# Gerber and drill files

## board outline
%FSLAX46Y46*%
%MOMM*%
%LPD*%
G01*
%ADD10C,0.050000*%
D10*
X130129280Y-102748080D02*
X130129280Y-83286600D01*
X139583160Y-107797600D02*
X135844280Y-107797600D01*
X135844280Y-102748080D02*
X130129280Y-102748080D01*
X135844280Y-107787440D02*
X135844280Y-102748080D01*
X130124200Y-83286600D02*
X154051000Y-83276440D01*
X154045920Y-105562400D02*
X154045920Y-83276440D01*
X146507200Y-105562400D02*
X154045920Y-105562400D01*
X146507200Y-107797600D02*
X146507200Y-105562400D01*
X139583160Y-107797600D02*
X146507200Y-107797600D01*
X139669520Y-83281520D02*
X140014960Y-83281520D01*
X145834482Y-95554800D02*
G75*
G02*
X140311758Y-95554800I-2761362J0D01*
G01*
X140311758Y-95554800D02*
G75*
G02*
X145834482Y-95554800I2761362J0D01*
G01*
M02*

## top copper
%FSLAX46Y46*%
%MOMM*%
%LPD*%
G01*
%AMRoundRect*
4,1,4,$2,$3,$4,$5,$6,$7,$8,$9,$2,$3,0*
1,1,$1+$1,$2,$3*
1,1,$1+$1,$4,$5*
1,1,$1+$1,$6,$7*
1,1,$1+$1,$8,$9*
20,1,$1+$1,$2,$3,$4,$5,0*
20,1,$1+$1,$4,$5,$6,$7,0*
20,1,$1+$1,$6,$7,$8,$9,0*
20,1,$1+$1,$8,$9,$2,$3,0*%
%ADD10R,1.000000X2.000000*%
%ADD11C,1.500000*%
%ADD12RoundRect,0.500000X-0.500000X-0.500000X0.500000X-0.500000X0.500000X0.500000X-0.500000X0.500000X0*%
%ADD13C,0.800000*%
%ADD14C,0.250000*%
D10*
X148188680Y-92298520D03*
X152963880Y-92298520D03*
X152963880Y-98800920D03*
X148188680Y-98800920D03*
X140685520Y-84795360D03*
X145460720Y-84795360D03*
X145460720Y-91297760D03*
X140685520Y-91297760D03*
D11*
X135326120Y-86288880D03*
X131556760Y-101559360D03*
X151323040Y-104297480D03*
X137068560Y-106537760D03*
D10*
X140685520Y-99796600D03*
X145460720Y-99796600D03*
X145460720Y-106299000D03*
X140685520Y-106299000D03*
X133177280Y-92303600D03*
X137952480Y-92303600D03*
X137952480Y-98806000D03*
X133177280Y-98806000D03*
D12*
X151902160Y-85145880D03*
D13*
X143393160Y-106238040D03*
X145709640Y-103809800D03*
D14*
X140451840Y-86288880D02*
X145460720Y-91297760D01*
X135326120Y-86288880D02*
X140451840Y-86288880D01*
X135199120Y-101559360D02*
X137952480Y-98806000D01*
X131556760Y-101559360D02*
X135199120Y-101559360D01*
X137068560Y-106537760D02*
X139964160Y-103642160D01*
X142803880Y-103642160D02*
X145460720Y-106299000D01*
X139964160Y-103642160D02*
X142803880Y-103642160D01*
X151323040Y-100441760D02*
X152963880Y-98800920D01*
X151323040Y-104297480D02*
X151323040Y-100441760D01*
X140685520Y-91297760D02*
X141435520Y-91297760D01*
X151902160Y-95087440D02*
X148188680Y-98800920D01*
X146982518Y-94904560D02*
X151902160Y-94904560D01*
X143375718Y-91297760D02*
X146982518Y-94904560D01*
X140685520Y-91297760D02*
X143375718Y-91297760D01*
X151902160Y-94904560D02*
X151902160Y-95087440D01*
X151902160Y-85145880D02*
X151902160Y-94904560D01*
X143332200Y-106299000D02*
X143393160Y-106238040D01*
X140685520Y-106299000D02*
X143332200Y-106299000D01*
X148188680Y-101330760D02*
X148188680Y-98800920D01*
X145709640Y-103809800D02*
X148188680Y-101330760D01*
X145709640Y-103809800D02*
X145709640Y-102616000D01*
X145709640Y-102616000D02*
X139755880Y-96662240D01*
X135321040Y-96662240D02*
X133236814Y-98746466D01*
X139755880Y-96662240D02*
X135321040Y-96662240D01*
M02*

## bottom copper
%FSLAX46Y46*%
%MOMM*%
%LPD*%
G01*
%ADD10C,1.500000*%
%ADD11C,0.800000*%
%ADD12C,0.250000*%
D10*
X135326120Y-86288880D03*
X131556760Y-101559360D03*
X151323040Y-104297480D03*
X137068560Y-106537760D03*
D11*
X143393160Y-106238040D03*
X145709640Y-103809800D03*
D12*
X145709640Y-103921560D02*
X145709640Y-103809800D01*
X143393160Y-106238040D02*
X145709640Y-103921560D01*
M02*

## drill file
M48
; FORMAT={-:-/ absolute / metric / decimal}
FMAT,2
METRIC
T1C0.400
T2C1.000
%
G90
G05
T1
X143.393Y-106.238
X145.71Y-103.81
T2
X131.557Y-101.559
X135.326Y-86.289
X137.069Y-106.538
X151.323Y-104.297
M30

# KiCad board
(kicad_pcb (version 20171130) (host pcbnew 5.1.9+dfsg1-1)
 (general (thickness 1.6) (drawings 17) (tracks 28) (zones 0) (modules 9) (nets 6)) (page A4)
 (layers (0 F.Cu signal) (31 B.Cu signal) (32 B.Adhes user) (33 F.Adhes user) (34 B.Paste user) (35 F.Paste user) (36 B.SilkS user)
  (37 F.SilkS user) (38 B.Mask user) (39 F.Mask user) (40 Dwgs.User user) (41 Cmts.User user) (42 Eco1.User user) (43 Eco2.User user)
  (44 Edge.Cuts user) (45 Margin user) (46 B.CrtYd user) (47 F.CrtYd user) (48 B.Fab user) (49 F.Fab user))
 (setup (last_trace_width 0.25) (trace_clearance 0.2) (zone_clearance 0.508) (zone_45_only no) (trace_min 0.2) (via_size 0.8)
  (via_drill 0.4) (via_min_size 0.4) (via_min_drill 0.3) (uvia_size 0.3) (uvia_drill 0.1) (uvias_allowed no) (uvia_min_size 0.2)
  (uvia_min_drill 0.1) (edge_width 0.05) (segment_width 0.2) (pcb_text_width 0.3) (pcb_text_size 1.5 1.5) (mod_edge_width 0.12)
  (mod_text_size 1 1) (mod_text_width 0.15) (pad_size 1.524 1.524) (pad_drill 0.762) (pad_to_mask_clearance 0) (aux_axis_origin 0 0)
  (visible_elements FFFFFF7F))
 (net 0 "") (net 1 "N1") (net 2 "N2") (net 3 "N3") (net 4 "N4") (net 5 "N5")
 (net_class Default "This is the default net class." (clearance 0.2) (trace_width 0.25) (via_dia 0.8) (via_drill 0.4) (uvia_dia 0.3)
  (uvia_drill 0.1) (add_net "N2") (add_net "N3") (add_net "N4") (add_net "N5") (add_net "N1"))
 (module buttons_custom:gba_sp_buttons (layer F.Cu) (at 150.57628 95.54972)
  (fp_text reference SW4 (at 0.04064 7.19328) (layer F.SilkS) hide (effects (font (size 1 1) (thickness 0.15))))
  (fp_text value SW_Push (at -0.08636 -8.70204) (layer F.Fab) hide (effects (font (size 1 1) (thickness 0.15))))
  (pad 3 smd rect (at -2.3876 -3.2512) (size 1 2) (layers F.Cu F.Paste F.Mask))
  (pad 4 smd rect (at 2.3876 -3.2512) (size 1 2) (layers F.Cu F.Paste F.Mask))
  (pad 2 smd rect (at 2.3876 3.2512) (size 1 2) (layers F.Cu F.Paste F.Mask) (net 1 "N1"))
  (pad 1 smd rect (at -2.3876 3.2512) (size 1 2) (layers F.Cu F.Paste F.Mask) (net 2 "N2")))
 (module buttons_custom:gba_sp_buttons (layer F.Cu) (at 143.07312 88.04656)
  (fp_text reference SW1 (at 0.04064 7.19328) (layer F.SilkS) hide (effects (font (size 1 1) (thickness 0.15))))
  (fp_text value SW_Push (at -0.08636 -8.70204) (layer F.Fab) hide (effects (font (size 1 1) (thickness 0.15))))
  (pad 3 smd rect (at -2.3876 -3.2512) (size 1 2) (layers F.Cu F.Paste F.Mask))
  (pad 4 smd rect (at 2.3876 -3.2512) (size 1 2) (layers F.Cu F.Paste F.Mask))
  (pad 2 smd rect (at 2.3876 3.2512) (size 1 2) (layers F.Cu F.Paste F.Mask) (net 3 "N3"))
  (pad 1 smd rect (at -2.3876 3.2512) (size 1 2) (layers F.Cu F.Paste F.Mask) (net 2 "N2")))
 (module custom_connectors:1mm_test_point (layer F.Cu) (at 135.32612 86.29904)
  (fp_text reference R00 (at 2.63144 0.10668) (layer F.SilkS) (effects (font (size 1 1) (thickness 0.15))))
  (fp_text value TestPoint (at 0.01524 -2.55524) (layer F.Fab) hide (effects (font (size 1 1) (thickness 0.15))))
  (pad 1 thru_hole circle (at 0 -0.01016) (size 1.5 1.5) (drill 1) (layers *.Cu *.Mask) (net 3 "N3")))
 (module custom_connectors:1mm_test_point (layer F.Cu) (at 131.55676 101.56952)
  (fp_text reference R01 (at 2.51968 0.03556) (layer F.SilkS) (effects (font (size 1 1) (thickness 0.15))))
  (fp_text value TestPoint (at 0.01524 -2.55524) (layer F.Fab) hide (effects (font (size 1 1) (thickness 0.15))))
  (pad 1 thru_hole circle (at 0 -0.01016) (size 1.5 1.5) (drill 1) (layers *.Cu *.Mask) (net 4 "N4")))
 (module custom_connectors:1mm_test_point (layer F.Cu) (at 151.32304 104.30764)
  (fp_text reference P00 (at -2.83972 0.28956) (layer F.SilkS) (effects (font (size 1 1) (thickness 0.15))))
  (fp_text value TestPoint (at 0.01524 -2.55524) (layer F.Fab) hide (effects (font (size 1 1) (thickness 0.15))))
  (pad 1 thru_hole circle (at 0 -0.01016) (size 1.5 1.5) (drill 1) (layers *.Cu *.Mask) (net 1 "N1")))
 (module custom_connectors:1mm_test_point (layer F.Cu) (at 137.06856 106.54792)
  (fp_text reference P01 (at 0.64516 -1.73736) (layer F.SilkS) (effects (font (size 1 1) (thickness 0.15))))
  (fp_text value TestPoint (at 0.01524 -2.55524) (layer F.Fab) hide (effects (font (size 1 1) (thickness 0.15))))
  (pad 1 thru_hole circle (at 0 -0.01016) (size 1.5 1.5) (drill 1) (layers *.Cu *.Mask) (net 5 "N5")))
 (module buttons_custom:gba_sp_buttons (layer F.Cu) (at 143.07312 103.0478)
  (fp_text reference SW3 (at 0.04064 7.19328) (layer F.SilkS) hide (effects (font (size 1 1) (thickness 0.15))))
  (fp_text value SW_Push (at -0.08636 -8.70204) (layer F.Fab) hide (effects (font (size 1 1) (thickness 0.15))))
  (pad 3 smd rect (at -2.3876 -3.2512) (size 1 2) (layers F.Cu F.Paste F.Mask))
  (pad 4 smd rect (at 2.3876 -3.2512) (size 1 2) (layers F.Cu F.Paste F.Mask))
  (pad 2 smd rect (at 2.3876 3.2512) (size 1 2) (layers F.Cu F.Paste F.Mask) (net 5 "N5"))
  (pad 1 smd rect (at -2.3876 3.2512) (size 1 2) (layers F.Cu F.Paste F.Mask) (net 2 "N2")))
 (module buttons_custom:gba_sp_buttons (layer F.Cu) (at 135.56488 95.5548)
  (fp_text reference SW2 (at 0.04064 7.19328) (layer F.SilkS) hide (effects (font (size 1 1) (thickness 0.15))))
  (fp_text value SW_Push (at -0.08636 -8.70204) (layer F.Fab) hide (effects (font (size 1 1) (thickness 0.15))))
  (pad 3 smd rect (at -2.3876 -3.2512) (size 1 2) (layers F.Cu F.Paste F.Mask))
  (pad 4 smd rect (at 2.3876 -3.2512) (size 1 2) (layers F.Cu F.Paste F.Mask))
  (pad 2 smd rect (at 2.3876 3.2512) (size 1 2) (layers F.Cu F.Paste F.Mask) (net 4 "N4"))
  (pad 1 smd rect (at -2.3876 3.2512) (size 1 2) (layers F.Cu F.Paste F.Mask) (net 2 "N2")))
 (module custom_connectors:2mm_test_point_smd (layer F.Cu) (at 151.90216 85.15604)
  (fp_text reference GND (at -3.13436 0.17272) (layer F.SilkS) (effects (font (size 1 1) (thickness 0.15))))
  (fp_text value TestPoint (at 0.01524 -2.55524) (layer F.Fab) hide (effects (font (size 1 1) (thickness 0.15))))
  (pad 1 smd roundrect (at 0 -0.01016) (size 2 2) (layers F.Cu F.Paste F.Mask) (roundrect_rratio 0.25) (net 2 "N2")))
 (gr_line (start 130.12928 102.74808) (end 130.12928 83.2866) (layer Edge.Cuts) (width 0.05))
 (gr_line (start 139.58316 107.7976) (end 135.84428 107.7976) (layer Edge.Cuts) (width 0.05))
 (gr_line (start 135.84428 102.74808) (end 130.12928 102.74808) (layer Edge.Cuts) (width 0.05))
 (gr_line (start 135.84428 107.78744) (end 135.84428 102.74808) (layer Edge.Cuts) (width 0.05))
 (gr_line (start 130.1242 83.2866) (end 154.051 83.27644) (layer Edge.Cuts) (width 0.05))
 (gr_line (start 154.04592 105.5624) (end 154.04592 83.27644) (layer Edge.Cuts) (width 0.05))
 (gr_line (start 146.5072 105.5624) (end 154.04592 105.5624) (layer Edge.Cuts) (width 0.05))
 (gr_line (start 146.5072 107.7976) (end 146.5072 105.5624) (layer Edge.Cuts) (width 0.05))
 (gr_line (start 139.58316 107.7976) (end 146.5072 107.7976) (layer Edge.Cuts) (width 0.05))
 (gr_line (start 139.66952 83.28152) (end 140.01496 83.28152) (layer Edge.Cuts) (width 0.05))
 (gr_circle (center 143.07312 95.5548) (end 145.83156 95.4278) (layer Edge.Cuts) (width 0.05))
 (segment (start 140.45184 86.28888) (end 145.46072 91.29776) (width 0.25) (layer F.Cu) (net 3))
 (segment (start 135.32612 86.28888) (end 140.45184 86.28888) (width 0.25) (layer F.Cu) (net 3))
 (segment (start 135.19912 101.55936) (end 137.95248 98.806) (width 0.25) (layer F.Cu) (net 4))
 (segment (start 131.55676 101.55936) (end 135.19912 101.55936) (width 0.25) (layer F.Cu) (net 4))
 (segment (start 137.06856 106.53776) (end 139.96416 103.64216) (width 0.25) (layer F.Cu) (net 5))
 (segment (start 142.80388 103.64216) (end 145.46072 106.299) (width 0.25) (layer F.Cu) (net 5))
 (segment (start 139.96416 103.64216) (end 142.80388 103.64216) (width 0.25) (layer F.Cu) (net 5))
 (segment (start 151.32304 100.44176) (end 152.96388 98.80092) (width 0.25) (layer F.Cu) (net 1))
 (segment (start 151.32304 104.29748) (end 151.32304 100.44176) (width 0.25) (layer F.Cu) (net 1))
 (segment (start 140.68552 91.29776) (end 141.43552 91.29776) (width 0.25) (layer F.Cu) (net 2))
 (segment (start 151.90216 95.08744) (end 148.18868 98.80092) (width 0.25) (layer F.Cu) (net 2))
 (segment (start 146.982518 94.90456) (end 151.90216 94.90456) (width 0.25) (layer F.Cu) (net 2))
 (segment (start 143.375718 91.29776) (end 146.982518 94.90456) (width 0.25) (layer F.Cu) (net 2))
 (segment (start 140.68552 91.29776) (end 143.375718 91.29776) (width 0.25) (layer F.Cu) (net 2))
 (segment (start 151.90216 94.90456) (end 151.90216 95.08744) (width 0.25) (layer F.Cu) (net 2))
 (segment (start 151.90216 85.14588) (end 151.90216 94.90456) (width 0.25) (layer F.Cu) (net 2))
 (via (at 143.39316 106.23804) (size 0.8) (drill 0.4) (layers F.Cu B.Cu) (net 2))
 (segment (start 143.3322 106.299) (end 143.39316 106.23804) (width 0.25) (layer F.Cu) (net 2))
 (segment (start 140.68552 106.299) (end 143.3322 106.299) (width 0.25) (layer F.Cu) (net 2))
 (via (at 145.70964 103.8098) (size 0.8) (drill 0.4) (layers F.Cu B.Cu) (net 2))
 (segment (start 145.70964 103.92156) (end 145.70964 103.8098) (width 0.25) (layer B.Cu) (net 2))
 (segment (start 143.39316 106.23804) (end 145.70964 103.92156) (width 0.25) (layer B.Cu) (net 2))
 (segment (start 148.18868 101.33076) (end 148.18868 98.80092) (width 0.25) (layer F.Cu) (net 2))
 (segment (start 145.70964 103.8098) (end 148.18868 101.33076) (width 0.25) (layer F.Cu) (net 2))
 (segment (start 145.70964 103.8098) (end 145.70964 102.616) (width 0.25) (layer F.Cu) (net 2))
 (segment (start 145.70964 102.616) (end 139.75588 96.66224) (width 0.25) (layer F.Cu) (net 2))
 (segment (start 135.32104 96.66224) (end 133.236814 98.746466) (width 0.25) (layer F.Cu) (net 2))
 (segment (start 139.75588 96.66224) (end 135.32104 96.66224) (width 0.25) (layer F.Cu) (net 2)))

